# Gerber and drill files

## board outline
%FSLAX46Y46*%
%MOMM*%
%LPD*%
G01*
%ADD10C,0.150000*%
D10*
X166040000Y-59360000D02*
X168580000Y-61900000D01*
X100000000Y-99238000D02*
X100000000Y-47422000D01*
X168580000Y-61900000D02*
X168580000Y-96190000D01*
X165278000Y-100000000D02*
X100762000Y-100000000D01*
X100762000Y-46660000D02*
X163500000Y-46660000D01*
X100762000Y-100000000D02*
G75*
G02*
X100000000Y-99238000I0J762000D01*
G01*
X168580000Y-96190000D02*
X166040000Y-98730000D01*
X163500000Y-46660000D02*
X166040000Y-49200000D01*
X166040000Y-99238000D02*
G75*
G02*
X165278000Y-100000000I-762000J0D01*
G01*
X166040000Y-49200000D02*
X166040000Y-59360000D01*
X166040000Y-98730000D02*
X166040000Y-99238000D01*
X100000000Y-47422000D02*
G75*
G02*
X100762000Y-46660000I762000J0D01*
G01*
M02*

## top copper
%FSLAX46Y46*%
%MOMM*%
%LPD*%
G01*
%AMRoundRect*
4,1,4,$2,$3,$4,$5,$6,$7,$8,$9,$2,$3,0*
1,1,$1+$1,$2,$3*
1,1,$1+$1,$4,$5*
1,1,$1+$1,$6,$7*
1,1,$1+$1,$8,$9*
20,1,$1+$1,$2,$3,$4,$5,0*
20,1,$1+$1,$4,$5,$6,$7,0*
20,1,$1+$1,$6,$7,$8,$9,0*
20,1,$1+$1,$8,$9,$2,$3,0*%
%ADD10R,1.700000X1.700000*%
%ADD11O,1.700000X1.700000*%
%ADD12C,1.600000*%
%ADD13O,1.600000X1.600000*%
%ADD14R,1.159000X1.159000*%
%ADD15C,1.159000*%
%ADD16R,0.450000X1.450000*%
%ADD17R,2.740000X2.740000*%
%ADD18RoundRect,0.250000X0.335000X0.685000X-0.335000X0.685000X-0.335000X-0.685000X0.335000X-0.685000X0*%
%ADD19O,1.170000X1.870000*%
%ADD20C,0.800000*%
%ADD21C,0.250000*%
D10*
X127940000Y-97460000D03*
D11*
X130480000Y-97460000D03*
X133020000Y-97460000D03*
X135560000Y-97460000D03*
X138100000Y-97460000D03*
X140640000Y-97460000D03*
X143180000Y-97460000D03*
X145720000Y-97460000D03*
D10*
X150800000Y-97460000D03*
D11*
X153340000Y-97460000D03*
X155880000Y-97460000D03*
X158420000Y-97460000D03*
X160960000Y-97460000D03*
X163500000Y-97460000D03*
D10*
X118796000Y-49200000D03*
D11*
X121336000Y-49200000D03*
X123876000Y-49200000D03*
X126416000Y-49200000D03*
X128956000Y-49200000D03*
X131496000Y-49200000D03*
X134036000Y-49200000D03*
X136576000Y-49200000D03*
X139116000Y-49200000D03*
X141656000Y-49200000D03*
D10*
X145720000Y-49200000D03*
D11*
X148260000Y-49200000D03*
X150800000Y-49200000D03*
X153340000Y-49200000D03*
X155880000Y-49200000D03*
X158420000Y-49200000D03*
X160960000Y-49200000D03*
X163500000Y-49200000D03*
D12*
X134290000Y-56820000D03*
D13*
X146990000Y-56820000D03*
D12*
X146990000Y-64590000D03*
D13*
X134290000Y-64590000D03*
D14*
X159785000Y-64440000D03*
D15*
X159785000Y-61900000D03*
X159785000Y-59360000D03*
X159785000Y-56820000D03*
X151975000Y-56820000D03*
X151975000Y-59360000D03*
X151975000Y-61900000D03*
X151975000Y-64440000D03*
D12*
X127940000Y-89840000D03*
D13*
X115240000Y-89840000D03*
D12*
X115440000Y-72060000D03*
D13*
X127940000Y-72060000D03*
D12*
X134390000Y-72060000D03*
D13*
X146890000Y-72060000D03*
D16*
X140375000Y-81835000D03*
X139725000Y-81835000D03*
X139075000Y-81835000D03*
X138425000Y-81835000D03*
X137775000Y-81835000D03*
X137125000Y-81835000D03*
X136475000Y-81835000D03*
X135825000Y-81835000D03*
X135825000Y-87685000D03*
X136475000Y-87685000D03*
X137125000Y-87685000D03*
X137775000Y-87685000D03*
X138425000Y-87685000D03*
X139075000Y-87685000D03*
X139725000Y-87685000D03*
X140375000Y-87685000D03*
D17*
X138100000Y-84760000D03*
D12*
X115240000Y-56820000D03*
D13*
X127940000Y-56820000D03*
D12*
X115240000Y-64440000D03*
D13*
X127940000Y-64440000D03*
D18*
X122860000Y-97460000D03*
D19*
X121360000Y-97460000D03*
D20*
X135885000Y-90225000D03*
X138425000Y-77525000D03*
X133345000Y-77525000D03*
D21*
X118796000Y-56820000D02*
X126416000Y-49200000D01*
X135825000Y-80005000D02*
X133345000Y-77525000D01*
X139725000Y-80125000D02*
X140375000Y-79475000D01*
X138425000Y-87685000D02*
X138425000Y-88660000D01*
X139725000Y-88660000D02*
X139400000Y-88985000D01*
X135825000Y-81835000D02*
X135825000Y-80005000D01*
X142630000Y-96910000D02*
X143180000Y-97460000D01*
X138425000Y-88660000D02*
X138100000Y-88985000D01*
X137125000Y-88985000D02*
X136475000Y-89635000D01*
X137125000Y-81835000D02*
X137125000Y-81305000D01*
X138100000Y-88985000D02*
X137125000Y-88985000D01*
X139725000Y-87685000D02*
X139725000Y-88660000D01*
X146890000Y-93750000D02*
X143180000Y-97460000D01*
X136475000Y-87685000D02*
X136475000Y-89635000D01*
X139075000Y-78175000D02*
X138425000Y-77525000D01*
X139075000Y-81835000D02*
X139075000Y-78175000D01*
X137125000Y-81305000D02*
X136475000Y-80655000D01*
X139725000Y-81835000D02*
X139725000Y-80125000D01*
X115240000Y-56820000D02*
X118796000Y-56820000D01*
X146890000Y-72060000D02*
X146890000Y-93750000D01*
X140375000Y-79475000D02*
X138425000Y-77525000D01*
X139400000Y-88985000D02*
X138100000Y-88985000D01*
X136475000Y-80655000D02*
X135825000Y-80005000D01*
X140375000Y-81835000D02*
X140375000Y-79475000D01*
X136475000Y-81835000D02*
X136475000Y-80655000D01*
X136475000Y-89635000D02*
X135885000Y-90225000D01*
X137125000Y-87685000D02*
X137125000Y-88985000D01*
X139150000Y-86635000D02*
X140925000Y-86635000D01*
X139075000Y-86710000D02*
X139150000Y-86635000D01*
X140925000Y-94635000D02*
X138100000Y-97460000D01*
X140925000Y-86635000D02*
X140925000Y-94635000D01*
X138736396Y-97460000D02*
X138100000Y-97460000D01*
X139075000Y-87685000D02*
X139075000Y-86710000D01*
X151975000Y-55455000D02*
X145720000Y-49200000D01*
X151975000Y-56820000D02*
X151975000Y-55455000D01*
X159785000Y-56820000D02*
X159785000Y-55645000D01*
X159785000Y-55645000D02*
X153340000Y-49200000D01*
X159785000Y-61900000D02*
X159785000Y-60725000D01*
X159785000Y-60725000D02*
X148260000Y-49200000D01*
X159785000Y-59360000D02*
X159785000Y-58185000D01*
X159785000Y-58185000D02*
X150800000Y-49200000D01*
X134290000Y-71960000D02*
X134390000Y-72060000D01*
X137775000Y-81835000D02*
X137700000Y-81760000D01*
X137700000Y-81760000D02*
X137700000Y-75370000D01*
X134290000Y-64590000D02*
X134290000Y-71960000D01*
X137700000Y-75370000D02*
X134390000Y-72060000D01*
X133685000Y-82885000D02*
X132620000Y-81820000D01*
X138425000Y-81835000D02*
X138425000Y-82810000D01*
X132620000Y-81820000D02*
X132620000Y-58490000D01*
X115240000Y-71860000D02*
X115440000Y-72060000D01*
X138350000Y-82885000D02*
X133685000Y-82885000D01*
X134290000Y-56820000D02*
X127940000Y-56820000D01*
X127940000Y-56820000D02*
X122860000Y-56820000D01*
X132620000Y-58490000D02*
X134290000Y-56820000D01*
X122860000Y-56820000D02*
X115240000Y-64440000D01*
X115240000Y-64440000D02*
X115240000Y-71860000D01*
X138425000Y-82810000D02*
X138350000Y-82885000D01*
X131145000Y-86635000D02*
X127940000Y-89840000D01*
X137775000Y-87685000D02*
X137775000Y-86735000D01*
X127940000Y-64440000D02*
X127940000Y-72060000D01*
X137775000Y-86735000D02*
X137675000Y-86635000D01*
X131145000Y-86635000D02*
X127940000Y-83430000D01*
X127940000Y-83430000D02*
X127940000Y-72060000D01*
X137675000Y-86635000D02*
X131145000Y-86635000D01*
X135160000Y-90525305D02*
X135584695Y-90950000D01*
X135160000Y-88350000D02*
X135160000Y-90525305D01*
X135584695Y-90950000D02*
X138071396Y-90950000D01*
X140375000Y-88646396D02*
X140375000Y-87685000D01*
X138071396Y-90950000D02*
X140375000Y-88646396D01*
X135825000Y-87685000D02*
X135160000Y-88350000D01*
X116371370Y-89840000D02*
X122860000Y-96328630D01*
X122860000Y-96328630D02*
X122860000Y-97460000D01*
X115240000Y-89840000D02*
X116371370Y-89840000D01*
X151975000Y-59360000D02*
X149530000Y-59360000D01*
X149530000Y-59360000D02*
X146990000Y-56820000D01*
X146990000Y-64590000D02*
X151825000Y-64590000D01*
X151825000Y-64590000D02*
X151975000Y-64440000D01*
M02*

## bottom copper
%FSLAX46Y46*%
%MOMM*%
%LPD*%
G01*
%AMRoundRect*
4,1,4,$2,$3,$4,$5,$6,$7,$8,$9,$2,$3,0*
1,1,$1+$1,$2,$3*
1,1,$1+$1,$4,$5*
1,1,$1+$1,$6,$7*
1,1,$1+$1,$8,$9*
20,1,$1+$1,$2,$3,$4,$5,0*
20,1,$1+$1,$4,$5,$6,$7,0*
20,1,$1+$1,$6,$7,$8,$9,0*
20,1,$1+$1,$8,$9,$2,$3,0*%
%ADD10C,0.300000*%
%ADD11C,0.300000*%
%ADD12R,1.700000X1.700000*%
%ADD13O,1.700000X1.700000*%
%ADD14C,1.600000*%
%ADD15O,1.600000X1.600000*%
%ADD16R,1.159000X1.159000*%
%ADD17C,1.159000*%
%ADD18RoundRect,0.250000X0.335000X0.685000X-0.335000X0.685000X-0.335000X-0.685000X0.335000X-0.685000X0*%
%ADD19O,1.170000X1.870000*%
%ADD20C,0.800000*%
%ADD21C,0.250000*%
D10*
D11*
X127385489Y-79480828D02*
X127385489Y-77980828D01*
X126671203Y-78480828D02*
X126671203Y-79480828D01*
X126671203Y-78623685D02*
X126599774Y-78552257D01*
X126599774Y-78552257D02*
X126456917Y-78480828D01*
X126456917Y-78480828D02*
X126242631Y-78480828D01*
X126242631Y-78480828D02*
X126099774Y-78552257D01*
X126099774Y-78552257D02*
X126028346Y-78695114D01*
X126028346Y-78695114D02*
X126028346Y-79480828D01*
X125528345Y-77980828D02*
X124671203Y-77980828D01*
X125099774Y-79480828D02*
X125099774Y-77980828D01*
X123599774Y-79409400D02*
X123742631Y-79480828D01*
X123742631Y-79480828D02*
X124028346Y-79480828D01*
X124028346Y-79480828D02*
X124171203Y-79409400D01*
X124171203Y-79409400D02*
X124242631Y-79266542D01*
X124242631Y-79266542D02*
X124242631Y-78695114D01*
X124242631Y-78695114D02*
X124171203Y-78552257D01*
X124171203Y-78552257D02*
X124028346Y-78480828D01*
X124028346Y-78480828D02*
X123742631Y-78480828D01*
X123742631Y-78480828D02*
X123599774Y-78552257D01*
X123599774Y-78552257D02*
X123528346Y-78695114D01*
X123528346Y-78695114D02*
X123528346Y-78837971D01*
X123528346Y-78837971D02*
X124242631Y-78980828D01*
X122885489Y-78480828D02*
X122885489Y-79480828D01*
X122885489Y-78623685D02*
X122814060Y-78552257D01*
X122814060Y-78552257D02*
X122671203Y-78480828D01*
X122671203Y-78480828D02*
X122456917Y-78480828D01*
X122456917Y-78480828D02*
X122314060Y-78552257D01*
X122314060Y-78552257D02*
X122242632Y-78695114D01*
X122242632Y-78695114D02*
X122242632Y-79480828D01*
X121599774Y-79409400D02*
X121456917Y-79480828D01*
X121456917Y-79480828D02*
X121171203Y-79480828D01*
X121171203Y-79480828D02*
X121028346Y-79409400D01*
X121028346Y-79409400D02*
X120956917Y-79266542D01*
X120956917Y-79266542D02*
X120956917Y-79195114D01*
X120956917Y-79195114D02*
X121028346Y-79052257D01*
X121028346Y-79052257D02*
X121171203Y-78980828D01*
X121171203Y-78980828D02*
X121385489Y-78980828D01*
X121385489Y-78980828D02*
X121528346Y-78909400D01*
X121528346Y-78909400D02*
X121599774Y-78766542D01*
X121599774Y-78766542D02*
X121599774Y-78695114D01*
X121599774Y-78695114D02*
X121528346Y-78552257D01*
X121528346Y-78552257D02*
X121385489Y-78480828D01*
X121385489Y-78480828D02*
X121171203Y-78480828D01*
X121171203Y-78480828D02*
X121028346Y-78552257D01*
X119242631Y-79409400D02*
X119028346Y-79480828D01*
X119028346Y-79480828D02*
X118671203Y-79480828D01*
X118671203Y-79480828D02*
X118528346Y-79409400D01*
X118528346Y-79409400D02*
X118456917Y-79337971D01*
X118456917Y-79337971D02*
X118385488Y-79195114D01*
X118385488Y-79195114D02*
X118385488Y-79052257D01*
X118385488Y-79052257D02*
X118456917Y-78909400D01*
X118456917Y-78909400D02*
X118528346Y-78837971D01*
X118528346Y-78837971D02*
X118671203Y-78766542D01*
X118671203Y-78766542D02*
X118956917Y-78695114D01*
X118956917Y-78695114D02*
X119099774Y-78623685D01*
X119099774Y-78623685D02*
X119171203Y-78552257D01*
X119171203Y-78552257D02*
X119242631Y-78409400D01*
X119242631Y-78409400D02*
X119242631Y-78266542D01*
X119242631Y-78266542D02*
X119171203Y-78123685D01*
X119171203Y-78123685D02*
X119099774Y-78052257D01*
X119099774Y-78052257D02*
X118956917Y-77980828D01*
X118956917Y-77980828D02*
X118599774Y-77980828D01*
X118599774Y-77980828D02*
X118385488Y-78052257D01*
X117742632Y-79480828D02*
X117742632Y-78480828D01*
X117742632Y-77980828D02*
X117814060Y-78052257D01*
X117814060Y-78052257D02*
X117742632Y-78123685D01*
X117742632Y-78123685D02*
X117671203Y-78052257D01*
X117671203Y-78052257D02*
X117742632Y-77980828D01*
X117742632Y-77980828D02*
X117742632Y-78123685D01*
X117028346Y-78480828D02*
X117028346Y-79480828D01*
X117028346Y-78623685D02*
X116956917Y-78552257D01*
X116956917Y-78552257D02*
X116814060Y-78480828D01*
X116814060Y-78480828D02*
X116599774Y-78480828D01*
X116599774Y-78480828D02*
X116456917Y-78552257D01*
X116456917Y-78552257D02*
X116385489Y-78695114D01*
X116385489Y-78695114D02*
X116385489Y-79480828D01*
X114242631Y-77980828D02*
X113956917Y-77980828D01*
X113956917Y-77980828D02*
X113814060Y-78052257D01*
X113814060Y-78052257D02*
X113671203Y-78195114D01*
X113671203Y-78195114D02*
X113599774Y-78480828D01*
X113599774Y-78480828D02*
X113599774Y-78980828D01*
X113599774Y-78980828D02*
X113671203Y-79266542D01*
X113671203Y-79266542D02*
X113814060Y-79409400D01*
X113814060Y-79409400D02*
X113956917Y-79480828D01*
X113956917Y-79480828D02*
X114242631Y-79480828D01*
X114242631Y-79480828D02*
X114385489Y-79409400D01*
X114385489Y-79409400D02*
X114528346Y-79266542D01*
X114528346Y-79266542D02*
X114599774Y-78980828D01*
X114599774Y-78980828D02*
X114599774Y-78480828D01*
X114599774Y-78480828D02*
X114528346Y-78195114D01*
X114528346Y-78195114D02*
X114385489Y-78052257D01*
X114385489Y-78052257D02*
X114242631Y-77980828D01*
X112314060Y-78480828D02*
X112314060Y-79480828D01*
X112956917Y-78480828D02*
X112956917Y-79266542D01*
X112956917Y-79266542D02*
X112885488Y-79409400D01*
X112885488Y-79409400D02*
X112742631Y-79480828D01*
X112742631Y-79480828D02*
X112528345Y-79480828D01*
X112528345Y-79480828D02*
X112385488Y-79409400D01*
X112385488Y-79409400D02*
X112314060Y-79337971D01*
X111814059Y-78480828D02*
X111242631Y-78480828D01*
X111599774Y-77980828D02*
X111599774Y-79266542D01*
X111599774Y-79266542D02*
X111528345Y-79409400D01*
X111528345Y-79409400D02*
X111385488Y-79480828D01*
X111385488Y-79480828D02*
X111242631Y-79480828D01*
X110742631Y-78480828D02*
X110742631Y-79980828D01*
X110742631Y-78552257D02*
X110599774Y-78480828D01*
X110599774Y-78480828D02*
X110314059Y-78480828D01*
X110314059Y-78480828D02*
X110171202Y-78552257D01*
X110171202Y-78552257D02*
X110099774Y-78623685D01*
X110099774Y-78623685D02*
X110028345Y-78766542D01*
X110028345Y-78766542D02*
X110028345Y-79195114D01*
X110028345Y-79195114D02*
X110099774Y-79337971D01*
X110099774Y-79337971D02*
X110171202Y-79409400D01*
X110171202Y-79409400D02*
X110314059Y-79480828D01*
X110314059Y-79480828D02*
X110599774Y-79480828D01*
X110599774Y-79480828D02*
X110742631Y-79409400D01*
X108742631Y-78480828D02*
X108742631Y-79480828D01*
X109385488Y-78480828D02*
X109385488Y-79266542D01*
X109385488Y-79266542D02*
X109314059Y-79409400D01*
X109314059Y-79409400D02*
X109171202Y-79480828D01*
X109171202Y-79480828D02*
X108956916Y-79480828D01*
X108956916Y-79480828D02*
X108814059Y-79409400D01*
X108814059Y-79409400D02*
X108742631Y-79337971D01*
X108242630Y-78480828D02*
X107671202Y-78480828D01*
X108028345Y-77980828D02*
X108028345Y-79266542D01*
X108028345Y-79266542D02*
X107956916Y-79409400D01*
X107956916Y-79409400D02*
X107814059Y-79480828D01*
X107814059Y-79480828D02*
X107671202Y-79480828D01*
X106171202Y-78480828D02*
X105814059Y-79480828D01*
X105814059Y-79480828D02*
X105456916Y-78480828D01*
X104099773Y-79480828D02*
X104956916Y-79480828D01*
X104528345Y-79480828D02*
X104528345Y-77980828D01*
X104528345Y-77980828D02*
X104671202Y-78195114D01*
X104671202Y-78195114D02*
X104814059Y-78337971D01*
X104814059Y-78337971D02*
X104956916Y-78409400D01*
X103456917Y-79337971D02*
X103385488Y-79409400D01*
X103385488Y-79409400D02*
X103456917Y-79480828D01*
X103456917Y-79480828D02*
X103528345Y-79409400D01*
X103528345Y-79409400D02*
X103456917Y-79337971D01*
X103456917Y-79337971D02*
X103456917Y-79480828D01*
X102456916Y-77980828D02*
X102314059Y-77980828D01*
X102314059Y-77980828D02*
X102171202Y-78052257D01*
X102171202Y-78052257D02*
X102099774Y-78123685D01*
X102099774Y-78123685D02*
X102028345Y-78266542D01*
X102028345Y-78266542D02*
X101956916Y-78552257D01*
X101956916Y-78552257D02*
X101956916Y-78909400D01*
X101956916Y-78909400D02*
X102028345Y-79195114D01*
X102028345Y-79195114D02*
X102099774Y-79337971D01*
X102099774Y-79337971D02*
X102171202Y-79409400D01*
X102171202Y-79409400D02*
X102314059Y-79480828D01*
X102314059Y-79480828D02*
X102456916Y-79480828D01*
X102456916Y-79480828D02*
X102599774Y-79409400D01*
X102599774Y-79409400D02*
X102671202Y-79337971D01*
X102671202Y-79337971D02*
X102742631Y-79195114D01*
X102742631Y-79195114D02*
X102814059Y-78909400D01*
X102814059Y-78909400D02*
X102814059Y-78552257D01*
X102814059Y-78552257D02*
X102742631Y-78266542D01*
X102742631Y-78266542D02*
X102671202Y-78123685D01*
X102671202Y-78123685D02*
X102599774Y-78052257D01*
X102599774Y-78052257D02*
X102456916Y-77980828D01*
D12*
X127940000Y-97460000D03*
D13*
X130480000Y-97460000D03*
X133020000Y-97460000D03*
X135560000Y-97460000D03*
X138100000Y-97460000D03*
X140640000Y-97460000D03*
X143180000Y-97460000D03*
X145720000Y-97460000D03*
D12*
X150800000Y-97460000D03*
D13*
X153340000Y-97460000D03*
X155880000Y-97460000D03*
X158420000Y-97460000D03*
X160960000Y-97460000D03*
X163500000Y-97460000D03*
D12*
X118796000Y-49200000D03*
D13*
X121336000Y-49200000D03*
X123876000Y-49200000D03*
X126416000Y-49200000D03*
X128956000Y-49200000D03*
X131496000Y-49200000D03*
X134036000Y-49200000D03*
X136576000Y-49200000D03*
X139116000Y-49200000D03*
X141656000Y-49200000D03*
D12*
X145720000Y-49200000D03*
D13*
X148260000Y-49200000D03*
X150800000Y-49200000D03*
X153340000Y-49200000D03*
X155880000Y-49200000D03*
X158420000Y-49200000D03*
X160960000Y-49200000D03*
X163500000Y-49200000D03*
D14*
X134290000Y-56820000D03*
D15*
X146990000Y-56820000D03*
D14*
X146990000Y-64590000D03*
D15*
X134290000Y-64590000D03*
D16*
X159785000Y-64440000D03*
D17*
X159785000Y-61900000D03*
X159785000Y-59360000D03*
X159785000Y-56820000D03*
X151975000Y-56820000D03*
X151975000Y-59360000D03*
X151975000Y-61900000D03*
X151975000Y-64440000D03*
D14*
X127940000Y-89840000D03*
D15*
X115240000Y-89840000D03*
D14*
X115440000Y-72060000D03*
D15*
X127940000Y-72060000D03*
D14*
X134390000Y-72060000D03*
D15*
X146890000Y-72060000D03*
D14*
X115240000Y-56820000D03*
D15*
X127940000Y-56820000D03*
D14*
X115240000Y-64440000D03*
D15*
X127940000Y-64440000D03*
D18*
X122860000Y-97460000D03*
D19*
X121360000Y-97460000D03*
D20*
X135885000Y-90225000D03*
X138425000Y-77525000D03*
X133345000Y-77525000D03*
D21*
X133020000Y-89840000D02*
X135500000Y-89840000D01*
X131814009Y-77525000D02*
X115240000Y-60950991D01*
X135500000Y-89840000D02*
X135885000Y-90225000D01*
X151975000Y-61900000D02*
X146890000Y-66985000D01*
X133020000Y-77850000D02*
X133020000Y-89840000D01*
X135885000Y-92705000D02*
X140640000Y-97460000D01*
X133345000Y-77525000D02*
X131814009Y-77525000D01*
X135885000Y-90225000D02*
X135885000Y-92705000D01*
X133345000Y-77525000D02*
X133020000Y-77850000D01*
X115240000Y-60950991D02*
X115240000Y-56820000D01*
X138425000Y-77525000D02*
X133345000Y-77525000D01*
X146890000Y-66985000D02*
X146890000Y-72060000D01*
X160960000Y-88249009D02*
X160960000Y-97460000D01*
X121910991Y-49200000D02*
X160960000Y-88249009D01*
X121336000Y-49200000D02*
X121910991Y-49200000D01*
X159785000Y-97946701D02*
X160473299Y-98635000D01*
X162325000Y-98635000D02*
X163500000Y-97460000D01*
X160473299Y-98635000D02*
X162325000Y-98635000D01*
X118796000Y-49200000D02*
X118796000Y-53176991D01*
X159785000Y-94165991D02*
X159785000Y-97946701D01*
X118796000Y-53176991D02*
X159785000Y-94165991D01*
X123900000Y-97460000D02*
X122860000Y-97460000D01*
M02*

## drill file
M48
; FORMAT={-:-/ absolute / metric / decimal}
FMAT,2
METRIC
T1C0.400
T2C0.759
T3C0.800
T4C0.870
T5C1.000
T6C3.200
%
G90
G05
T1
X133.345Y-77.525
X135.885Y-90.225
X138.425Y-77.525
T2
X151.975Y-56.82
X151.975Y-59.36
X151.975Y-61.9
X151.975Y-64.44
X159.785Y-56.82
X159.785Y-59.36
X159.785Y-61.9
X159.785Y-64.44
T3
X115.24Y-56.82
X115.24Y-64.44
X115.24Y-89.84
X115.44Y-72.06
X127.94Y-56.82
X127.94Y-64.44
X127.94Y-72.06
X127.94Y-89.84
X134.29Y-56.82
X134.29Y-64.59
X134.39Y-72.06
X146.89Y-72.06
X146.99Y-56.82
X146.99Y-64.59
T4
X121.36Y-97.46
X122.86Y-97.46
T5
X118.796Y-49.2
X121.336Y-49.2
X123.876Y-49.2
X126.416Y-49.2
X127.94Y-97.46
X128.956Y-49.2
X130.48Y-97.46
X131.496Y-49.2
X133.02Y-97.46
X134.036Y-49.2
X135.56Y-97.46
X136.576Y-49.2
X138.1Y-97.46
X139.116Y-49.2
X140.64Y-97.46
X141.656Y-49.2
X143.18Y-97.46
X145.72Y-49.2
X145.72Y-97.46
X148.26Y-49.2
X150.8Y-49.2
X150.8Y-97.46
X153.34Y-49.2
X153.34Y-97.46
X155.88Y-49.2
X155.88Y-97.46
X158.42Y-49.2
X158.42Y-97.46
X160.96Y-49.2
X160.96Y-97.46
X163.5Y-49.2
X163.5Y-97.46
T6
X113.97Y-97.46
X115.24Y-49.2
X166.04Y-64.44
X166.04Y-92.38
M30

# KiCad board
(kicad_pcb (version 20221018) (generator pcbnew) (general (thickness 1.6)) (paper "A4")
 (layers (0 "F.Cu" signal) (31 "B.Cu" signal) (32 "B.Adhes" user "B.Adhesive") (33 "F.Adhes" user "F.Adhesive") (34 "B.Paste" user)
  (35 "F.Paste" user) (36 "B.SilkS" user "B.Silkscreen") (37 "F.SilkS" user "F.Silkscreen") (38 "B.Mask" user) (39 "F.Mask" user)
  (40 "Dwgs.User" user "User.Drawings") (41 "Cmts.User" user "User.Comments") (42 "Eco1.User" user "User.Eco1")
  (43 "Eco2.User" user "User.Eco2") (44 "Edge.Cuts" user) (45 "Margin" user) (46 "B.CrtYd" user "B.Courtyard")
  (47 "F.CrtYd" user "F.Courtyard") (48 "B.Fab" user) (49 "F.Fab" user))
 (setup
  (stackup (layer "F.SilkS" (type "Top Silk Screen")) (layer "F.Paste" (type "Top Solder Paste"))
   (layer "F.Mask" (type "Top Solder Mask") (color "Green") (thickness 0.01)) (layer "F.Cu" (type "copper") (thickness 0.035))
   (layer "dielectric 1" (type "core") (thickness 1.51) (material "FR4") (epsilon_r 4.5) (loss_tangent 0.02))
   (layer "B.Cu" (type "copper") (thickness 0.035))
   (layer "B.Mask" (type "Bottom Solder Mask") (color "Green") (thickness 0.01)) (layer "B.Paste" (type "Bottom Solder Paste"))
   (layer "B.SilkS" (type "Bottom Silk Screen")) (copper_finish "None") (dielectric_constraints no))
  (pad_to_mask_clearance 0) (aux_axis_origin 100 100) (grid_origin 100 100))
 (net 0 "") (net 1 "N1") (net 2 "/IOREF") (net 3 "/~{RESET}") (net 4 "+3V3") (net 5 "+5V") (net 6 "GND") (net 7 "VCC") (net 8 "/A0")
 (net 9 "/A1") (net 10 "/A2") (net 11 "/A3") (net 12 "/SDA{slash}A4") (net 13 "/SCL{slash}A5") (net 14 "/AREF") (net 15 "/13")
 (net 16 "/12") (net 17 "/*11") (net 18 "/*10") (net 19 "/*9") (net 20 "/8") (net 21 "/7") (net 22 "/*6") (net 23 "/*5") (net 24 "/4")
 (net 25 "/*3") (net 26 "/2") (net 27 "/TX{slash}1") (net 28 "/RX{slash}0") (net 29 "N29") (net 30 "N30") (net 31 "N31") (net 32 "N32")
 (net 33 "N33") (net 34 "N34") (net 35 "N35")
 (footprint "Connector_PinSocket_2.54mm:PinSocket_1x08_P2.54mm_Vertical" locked (layer "F.Cu") (at 127.94 97.46 90)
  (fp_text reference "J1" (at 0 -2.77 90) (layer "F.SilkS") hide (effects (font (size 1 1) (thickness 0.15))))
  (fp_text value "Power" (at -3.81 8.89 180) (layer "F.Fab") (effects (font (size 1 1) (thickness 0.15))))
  (pad "1" thru_hole rect locked (at 0 0 90) (size 1.7 1.7) (drill 1) (layers "*.Cu" "*.Mask") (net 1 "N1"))
  (pad "2" thru_hole oval locked (at 0 2.54 90) (size 1.7 1.7) (drill 1) (layers "*.Cu" "*.Mask") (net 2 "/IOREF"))
  (pad "3" thru_hole oval locked (at 0 5.08 90) (size 1.7 1.7) (drill 1) (layers "*.Cu" "*.Mask") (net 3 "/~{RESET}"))
  (pad "4" thru_hole oval locked (at 0 7.62 90) (size 1.7 1.7) (drill 1) (layers "*.Cu" "*.Mask") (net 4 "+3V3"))
  (pad "5" thru_hole oval locked (at 0 10.16 90) (size 1.7 1.7) (drill 1) (layers "*.Cu" "*.Mask") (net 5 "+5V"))
  (pad "6" thru_hole oval locked (at 0 12.7 90) (size 1.7 1.7) (drill 1) (layers "*.Cu" "*.Mask") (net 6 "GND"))
  (pad "7" thru_hole oval locked (at 0 15.24 90) (size 1.7 1.7) (drill 1) (layers "*.Cu" "*.Mask") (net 6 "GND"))
  (pad "8" thru_hole oval locked (at 0 17.78 90) (size 1.7 1.7) (drill 1) (layers "*.Cu" "*.Mask") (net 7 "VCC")))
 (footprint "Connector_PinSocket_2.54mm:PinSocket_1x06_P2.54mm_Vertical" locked (layer "F.Cu") (at 150.8 97.46 90)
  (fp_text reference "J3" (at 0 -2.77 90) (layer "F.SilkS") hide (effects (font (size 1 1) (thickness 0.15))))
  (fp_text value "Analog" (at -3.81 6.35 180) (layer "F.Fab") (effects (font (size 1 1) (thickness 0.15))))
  (pad "1" thru_hole rect locked (at 0 0 90) (size 1.7 1.7) (drill 1) (layers "*.Cu" "*.Mask") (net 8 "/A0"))
  (pad "2" thru_hole oval locked (at 0 2.54 90) (size 1.7 1.7) (drill 1) (layers "*.Cu" "*.Mask") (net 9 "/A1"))
  (pad "3" thru_hole oval locked (at 0 5.08 90) (size 1.7 1.7) (drill 1) (layers "*.Cu" "*.Mask") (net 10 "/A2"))
  (pad "4" thru_hole oval locked (at 0 7.62 90) (size 1.7 1.7) (drill 1) (layers "*.Cu" "*.Mask") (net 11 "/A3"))
  (pad "5" thru_hole oval locked (at 0 10.16 90) (size 1.7 1.7) (drill 1) (layers "*.Cu" "*.Mask") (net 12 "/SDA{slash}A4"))
  (pad "6" thru_hole oval locked (at 0 12.7 90) (size 1.7 1.7) (drill 1) (layers "*.Cu" "*.Mask") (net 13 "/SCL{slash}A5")))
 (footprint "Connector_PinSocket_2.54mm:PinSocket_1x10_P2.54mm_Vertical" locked (layer "F.Cu") (at 118.796 49.2 90)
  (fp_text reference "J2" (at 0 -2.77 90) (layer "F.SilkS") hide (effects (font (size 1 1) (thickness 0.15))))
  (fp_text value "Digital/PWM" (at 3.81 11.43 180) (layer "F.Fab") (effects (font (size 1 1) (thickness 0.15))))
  (pad "1" thru_hole rect locked (at 0 0 90) (size 1.7 1.7) (drill 1) (layers "*.Cu" "*.Mask") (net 13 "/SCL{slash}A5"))
  (pad "2" thru_hole oval locked (at 0 2.54 90) (size 1.7 1.7) (drill 1) (layers "*.Cu" "*.Mask") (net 12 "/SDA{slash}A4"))
  (pad "3" thru_hole oval locked (at 0 5.08 90) (size 1.7 1.7) (drill 1) (layers "*.Cu" "*.Mask") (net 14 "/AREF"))
  (pad "4" thru_hole oval locked (at 0 7.62 90) (size 1.7 1.7) (drill 1) (layers "*.Cu" "*.Mask") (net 6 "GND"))
  (pad "5" thru_hole oval locked (at 0 10.16 90) (size 1.7 1.7) (drill 1) (layers "*.Cu" "*.Mask") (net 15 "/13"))
  (pad "6" thru_hole oval locked (at 0 12.7 90) (size 1.7 1.7) (drill 1) (layers "*.Cu" "*.Mask") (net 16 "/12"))
  (pad "7" thru_hole oval locked (at 0 15.24 90) (size 1.7 1.7) (drill 1) (layers "*.Cu" "*.Mask") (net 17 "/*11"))
  (pad "8" thru_hole oval locked (at 0 17.78 90) (size 1.7 1.7) (drill 1) (layers "*.Cu" "*.Mask") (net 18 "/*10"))
  (pad "9" thru_hole oval locked (at 0 20.32 90) (size 1.7 1.7) (drill 1) (layers "*.Cu" "*.Mask") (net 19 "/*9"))
  (pad "10" thru_hole oval locked (at 0 22.86 90) (size 1.7 1.7) (drill 1) (layers "*.Cu" "*.Mask") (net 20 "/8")))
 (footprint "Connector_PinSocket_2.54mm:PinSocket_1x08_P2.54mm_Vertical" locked (layer "F.Cu") (at 145.72 49.2 90)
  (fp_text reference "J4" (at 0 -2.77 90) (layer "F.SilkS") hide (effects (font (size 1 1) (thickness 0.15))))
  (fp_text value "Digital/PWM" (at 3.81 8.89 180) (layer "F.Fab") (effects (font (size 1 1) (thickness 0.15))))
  (pad "1" thru_hole rect locked (at 0 0 90) (size 1.7 1.7) (drill 1) (layers "*.Cu" "*.Mask") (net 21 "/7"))
  (pad "2" thru_hole oval locked (at 0 2.54 90) (size 1.7 1.7) (drill 1) (layers "*.Cu" "*.Mask") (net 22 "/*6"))
  (pad "3" thru_hole oval locked (at 0 5.08 90) (size 1.7 1.7) (drill 1) (layers "*.Cu" "*.Mask") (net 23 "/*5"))
  (pad "4" thru_hole oval locked (at 0 7.62 90) (size 1.7 1.7) (drill 1) (layers "*.Cu" "*.Mask") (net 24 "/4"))
  (pad "5" thru_hole oval locked (at 0 10.16 90) (size 1.7 1.7) (drill 1) (layers "*.Cu" "*.Mask") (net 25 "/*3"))
  (pad "6" thru_hole oval locked (at 0 12.7 90) (size 1.7 1.7) (drill 1) (layers "*.Cu" "*.Mask") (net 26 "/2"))
  (pad "7" thru_hole oval locked (at 0 15.24 90) (size 1.7 1.7) (drill 1) (layers "*.Cu" "*.Mask") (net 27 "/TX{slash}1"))
  (pad "8" thru_hole oval locked (at 0 17.78 90) (size 1.7 1.7) (drill 1) (layers "*.Cu" "*.Mask") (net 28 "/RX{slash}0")))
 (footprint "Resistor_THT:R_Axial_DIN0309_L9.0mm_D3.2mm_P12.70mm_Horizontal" (layer "F.Cu") (at 134.29 56.82)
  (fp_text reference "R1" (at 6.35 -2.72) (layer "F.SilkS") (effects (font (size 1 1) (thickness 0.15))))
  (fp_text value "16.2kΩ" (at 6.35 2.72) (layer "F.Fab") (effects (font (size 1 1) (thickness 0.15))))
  (pad "1" thru_hole circle (at 0 0) (size 1.6 1.6) (drill 0.8) (layers "*.Cu" "*.Mask") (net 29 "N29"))
  (pad "2" thru_hole oval (at 12.7 0) (size 1.6 1.6) (drill 0.8) (layers "*.Cu" "*.Mask") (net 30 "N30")))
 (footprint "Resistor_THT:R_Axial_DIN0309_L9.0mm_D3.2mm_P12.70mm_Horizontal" (layer "F.Cu") (at 146.99 64.59 180)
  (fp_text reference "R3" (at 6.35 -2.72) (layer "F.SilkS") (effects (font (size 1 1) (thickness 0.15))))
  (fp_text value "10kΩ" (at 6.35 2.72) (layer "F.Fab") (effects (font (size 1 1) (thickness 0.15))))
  (pad "1" thru_hole circle (at 0 0 180) (size 1.6 1.6) (drill 0.8) (layers "*.Cu" "*.Mask") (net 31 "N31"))
  (pad "2" thru_hole oval (at 12.7 0 180) (size 1.6 1.6) (drill 0.8) (layers "*.Cu" "*.Mask") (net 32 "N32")))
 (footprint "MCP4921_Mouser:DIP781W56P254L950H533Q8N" (layer "F.Cu") (at 155.88 60.63 180)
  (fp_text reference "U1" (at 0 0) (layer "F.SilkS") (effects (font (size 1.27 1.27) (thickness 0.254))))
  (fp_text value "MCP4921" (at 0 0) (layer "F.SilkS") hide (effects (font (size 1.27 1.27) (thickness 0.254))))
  (pad "1" thru_hole rect (at -3.905 -3.81 180) (size 1.159 1.159) (drill 0.759) (layers "*.Cu" "*.Mask") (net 5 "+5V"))
  (pad "2" thru_hole circle (at -3.905 -1.27 180) (size 1.159 1.159) (drill 0.759) (layers "*.Cu" "*.Mask") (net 22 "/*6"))
  (pad "3" thru_hole circle (at -3.905 1.27 180) (size 1.159 1.159) (drill 0.759) (layers "*.Cu" "*.Mask") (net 23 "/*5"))
  (pad "4" thru_hole circle (at -3.905 3.81 180) (size 1.159 1.159) (drill 0.759) (layers "*.Cu" "*.Mask") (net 24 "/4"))
  (pad "5" thru_hole circle (at 3.905 3.81 180) (size 1.159 1.159) (drill 0.759) (layers "*.Cu" "*.Mask") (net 21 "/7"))
  (pad "6" thru_hole circle (at 3.905 1.27 180) (size 1.159 1.159) (drill 0.759) (layers "*.Cu" "*.Mask") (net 30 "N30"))
  (pad "7" thru_hole circle (at 3.905 -1.27 180) (size 1.159 1.159) (drill 0.759) (layers "*.Cu" "*.Mask") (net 6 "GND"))
  (pad "8" thru_hole circle (at 3.905 -3.81 180) (size 1.159 1.159) (drill 0.759) (layers "*.Cu" "*.Mask") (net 31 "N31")))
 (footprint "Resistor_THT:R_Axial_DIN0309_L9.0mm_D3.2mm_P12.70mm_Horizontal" (layer "F.Cu") (at 127.94 89.84 180)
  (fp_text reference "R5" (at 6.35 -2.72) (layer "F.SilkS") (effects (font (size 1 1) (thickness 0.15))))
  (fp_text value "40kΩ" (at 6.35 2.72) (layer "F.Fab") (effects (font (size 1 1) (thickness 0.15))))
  (pad "1" thru_hole circle (at 0 0 180) (size 1.6 1.6) (drill 0.8) (layers "*.Cu" "*.Mask") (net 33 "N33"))
  (pad "2" thru_hole oval (at 12.7 0 180) (size 1.6 1.6) (drill 0.8) (layers "*.Cu" "*.Mask") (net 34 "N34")))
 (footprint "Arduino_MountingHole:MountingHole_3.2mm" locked (layer "F.Cu") (at 115.24 49.2)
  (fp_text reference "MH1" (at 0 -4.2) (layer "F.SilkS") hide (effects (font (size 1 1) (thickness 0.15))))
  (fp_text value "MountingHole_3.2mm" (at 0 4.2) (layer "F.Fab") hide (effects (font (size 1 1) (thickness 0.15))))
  (pad "" np_thru_hole circle locked (at 0 0) (size 3.2 3.2) (drill 3.2) (layers "*.Cu" "*.Mask")))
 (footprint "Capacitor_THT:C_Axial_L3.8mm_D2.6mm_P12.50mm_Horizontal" (layer "F.Cu") (at 115.44 72.06)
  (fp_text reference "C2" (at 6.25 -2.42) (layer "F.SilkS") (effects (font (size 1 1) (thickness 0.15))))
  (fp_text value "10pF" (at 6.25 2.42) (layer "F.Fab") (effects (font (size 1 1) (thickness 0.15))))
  (pad "1" thru_hole circle (at 0 0) (size 1.6 1.6) (drill 0.8) (layers "*.Cu" "*.Mask") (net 29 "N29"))
  (pad "2" thru_hole oval (at 12.5 0) (size 1.6 1.6) (drill 0.8) (layers "*.Cu" "*.Mask") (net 33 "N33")))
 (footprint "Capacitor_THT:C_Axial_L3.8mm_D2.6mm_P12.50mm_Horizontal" (layer "F.Cu") (at 134.39 72.06)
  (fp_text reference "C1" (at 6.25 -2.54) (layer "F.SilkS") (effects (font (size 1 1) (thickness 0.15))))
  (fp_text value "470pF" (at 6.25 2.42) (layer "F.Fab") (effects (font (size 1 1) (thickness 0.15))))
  (pad "1" thru_hole circle (at 0 0) (size 1.6 1.6) (drill 0.8) (layers "*.Cu" "*.Mask") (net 32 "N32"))
  (pad "2" thru_hole oval (at 12.5 0) (size 1.6 1.6) (drill 0.8) (layers "*.Cu" "*.Mask") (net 6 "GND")))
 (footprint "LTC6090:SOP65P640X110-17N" (layer "F.Cu") (at 138.1 84.76 -90)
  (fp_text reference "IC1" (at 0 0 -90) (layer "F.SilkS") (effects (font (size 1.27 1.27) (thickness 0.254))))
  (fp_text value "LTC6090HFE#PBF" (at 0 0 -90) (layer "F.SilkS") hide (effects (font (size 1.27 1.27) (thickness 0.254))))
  (pad "1" smd rect (at -2.925 -2.275) (size 0.45 1.45) (layers "F.Cu" "F.Paste" "F.Mask") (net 6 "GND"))
  (pad "2" smd rect (at -2.925 -1.625) (size 0.45 1.45) (layers "F.Cu" "F.Paste" "F.Mask") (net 6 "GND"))
  (pad "3" smd rect (at -2.925 -0.975) (size 0.45 1.45) (layers "F.Cu" "F.Paste" "F.Mask") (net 6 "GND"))
  (pad "4" smd rect (at -2.925 -0.325) (size 0.45 1.45) (layers "F.Cu" "F.Paste" "F.Mask") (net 29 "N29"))
  (pad "5" smd rect (at -2.925 0.325) (size 0.45 1.45) (layers "F.Cu" "F.Paste" "F.Mask") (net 32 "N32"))
  (pad "6" smd rect (at -2.925 0.975) (size 0.45 1.45) (layers "F.Cu" "F.Paste" "F.Mask") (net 6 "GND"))
  (pad "7" smd rect (at -2.925 1.625) (size 0.45 1.45) (layers "F.Cu" "F.Paste" "F.Mask") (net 6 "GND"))
  (pad "8" smd rect (at -2.925 2.275) (size 0.45 1.45) (layers "F.Cu" "F.Paste" "F.Mask") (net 6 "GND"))
  (pad "9" smd rect (at 2.925 2.275) (size 0.45 1.45) (layers "F.Cu" "F.Paste" "F.Mask") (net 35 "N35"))
  (pad "10" smd rect (at 2.925 1.625) (size 0.45 1.45) (layers "F.Cu" "F.Paste" "F.Mask") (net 6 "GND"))
  (pad "11" smd rect (at 2.925 0.975) (size 0.45 1.45) (layers "F.Cu" "F.Paste" "F.Mask") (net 6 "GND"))
  (pad "12" smd rect (at 2.925 0.325) (size 0.45 1.45) (layers "F.Cu" "F.Paste" "F.Mask") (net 33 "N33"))
  (pad "13" smd rect (at 2.925 -0.325) (size 0.45 1.45) (layers "F.Cu" "F.Paste" "F.Mask") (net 6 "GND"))
  (pad "14" smd rect (at 2.925 -0.975) (size 0.45 1.45) (layers "F.Cu" "F.Paste" "F.Mask") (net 5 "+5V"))
  (pad "15" smd rect (at 2.925 -1.625) (size 0.45 1.45) (layers "F.Cu" "F.Paste" "F.Mask") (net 6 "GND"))
  (pad "16" smd rect (at 2.925 -2.275) (size 0.45 1.45) (layers "F.Cu" "F.Paste" "F.Mask") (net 35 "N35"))
  (pad "17" smd rect (at 0 0 270) (size 2.74 2.74) (layers "F.Cu" "F.Paste" "F.Mask") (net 6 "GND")))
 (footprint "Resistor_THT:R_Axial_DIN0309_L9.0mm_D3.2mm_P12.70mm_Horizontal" (layer "F.Cu") (at 115.24 56.82)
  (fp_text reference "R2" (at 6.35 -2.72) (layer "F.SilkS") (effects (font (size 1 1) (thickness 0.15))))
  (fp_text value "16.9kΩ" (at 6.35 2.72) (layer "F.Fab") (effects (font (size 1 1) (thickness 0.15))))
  (pad "1" thru_hole circle (at 0 0) (size 1.6 1.6) (drill 0.8) (layers "*.Cu" "*.Mask") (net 6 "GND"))
  (pad "2" thru_hole oval (at 12.7 0) (size 1.6 1.6) (drill 0.8) (layers "*.Cu" "*.Mask") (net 29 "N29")))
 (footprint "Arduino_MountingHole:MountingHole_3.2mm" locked (layer "F.Cu") (at 113.97 97.46)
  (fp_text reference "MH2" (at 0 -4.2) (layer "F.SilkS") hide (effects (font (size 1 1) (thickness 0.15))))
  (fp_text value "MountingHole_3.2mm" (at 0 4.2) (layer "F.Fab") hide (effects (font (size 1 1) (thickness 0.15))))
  (pad "" np_thru_hole circle locked (at 0 0) (size 3.2 3.2) (drill 3.2) (layers "*.Cu" "*.Mask")))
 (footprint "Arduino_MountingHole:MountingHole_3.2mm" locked (layer "F.Cu") (at 166.04 64.44)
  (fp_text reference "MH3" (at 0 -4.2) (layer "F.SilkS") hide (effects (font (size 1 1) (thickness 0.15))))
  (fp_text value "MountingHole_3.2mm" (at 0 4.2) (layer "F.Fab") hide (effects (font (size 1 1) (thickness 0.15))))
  (pad "" np_thru_hole circle locked (at 0 0) (size 3.2 3.2) (drill 3.2) (layers "*.Cu" "*.Mask")))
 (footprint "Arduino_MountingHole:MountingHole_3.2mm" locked (layer "F.Cu") (at 166.04 92.38)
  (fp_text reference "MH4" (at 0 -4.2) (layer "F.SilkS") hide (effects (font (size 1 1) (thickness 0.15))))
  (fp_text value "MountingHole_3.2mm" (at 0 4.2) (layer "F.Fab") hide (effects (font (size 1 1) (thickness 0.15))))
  (pad "" np_thru_hole circle locked (at 0 0) (size 3.2 3.2) (drill 3.2) (layers "*.Cu" "*.Mask")))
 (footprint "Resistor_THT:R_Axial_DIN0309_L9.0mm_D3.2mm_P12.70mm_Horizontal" (layer "F.Cu") (at 115.24 64.44)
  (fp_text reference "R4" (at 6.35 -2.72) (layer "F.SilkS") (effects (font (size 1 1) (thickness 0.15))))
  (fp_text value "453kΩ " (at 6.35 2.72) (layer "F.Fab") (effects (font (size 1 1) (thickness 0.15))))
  (pad "1" thru_hole circle (at 0 0) (size 1.6 1.6) (drill 0.8) (layers "*.Cu" "*.Mask") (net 29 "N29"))
  (pad "2" thru_hole oval (at 12.7 0) (size 1.6 1.6) (drill 0.8) (layers "*.Cu" "*.Mask") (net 33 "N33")))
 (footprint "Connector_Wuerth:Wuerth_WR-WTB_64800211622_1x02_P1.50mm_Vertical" (layer "B.Cu") (at 122.86 97.46 180)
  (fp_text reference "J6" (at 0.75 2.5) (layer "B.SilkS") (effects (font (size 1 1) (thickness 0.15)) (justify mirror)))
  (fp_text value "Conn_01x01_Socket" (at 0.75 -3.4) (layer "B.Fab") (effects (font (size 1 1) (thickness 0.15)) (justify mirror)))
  (pad "1" thru_hole roundrect (at 0 0 180) (size 1.17 1.87) (drill 0.87) (layers "*.Cu" "*.Mask") (roundrect_rratio 0.213675)
   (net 34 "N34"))
  (pad "2" thru_hole oval (at 1.5 0 180) (size 1.17 1.87) (drill 0.87) (layers "*.Cu" "*.Mask")))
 (gr_line (start 166.04 59.36) (end 168.58 61.9) (stroke (width 0.15) (type solid)) (layer "Edge.Cuts"))
 (gr_line (start 100 99.238) (end 100 47.422) (stroke (width 0.15) (type solid)) (layer "Edge.Cuts"))
 (gr_line (start 168.58 61.9) (end 168.58 96.19) (stroke (width 0.15) (type solid)) (layer "Edge.Cuts"))
 (gr_line (start 165.278 100) (end 100.762 100) (stroke (width 0.15) (type solid)) (layer "Edge.Cuts"))
 (gr_line (start 100.762 46.66) (end 163.5 46.66) (stroke (width 0.15) (type solid)) (layer "Edge.Cuts"))
 (gr_arc (start 100.762 100) (mid 100.223185 99.776815) (end 100 99.238) (stroke (width 0.15) (type solid)) (layer "Edge.Cuts"))
 (gr_line (start 168.58 96.19) (end 166.04 98.73) (stroke (width 0.15) (type solid)) (layer "Edge.Cuts"))
 (gr_line (start 163.5 46.66) (end 166.04 49.2) (stroke (width 0.15) (type solid)) (layer "Edge.Cuts"))
 (gr_arc (start 166.04 99.238) (mid 165.816815 99.776815) (end 165.278 100) (stroke (width 0.15) (type solid)) (layer "Edge.Cuts"))
 (gr_line (start 166.04 49.2) (end 166.04 59.36) (stroke (width 0.15) (type solid)) (layer "Edge.Cuts"))
 (gr_line (start 166.04 98.73) (end 166.04 99.238) (stroke (width 0.15) (type solid)) (layer "Edge.Cuts"))
 (gr_arc (start 100 47.422) (mid 100.223185 46.883185) (end 100.762 46.66) (stroke (width 0.15) (type solid)) (layer "Edge.Cuts"))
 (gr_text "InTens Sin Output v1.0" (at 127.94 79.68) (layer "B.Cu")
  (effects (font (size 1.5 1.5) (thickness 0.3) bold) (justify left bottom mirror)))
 (segment (start 118.796 56.82) (end 126.416 49.2) (width 0.25) (layer "F.Cu") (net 6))
 (segment (start 135.825 80.005) (end 133.345 77.525) (width 0.25) (layer "F.Cu") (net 6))
 (segment (start 139.725 80.125) (end 140.375 79.475) (width 0.25) (layer "F.Cu") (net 6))
 (segment (start 138.425 87.685) (end 138.425 88.66) (width 0.25) (layer "F.Cu") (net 6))
 (segment (start 139.725 88.66) (end 139.4 88.985) (width 0.25) (layer "F.Cu") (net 6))
 (segment (start 135.825 81.835) (end 135.825 80.005) (width 0.25) (layer "F.Cu") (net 6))
 (segment (start 142.63 96.91) (end 143.18 97.46) (width 0.25) (layer "F.Cu") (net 6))
 (segment (start 138.425 88.66) (end 138.1 88.985) (width 0.25) (layer "F.Cu") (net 6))
 (segment (start 137.125 88.985) (end 136.475 89.635) (width 0.25) (layer "F.Cu") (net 6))
 (segment (start 137.125 81.835) (end 137.125 81.305) (width 0.25) (layer "F.Cu") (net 6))
 (segment (start 138.1 88.985) (end 137.125 88.985) (width 0.25) (layer "F.Cu") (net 6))
 (segment (start 139.725 87.685) (end 139.725 88.66) (width 0.25) (layer "F.Cu") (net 6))
 (segment (start 146.89 93.75) (end 143.18 97.46) (width 0.25) (layer "F.Cu") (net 6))
 (segment (start 136.475 87.685) (end 136.475 89.635) (width 0.25) (layer "F.Cu") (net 6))
 (segment (start 139.075 78.175) (end 138.425 77.525) (width 0.25) (layer "F.Cu") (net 6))
 (segment (start 139.075 81.835) (end 139.075 78.175) (width 0.25) (layer "F.Cu") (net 6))
 (segment (start 137.125 81.305) (end 136.475 80.655) (width 0.25) (layer "F.Cu") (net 6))
 (segment (start 139.725 81.835) (end 139.725 80.125) (width 0.25) (layer "F.Cu") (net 6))
 (segment (start 115.24 56.82) (end 118.796 56.82) (width 0.25) (layer "F.Cu") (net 6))
 (segment (start 146.89 72.06) (end 146.89 93.75) (width 0.25) (layer "F.Cu") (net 6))
 (segment (start 140.375 79.475) (end 138.425 77.525) (width 0.25) (layer "F.Cu") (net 6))
 (segment (start 139.4 88.985) (end 138.1 88.985) (width 0.25) (layer "F.Cu") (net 6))
 (segment (start 136.475 80.655) (end 135.825 80.005) (width 0.25) (layer "F.Cu") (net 6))
 (segment (start 140.375 81.835) (end 140.375 79.475) (width 0.25) (layer "F.Cu") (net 6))
 (segment (start 136.475 81.835) (end 136.475 80.655) (width 0.25) (layer "F.Cu") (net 6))
 (segment (start 136.475 89.635) (end 135.885 90.225) (width 0.25) (layer "F.Cu") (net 6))
 (segment (start 137.125 87.685) (end 137.125 88.985) (width 0.25) (layer "F.Cu") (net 6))
 (via (at 135.885 90.225) (size 0.8) (drill 0.4) (layers "F.Cu" "B.Cu") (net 6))
 (via (at 138.425 77.525) (size 0.8) (drill 0.4) (layers "F.Cu" "B.Cu") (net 6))
 (via (at 133.345 77.525) (size 0.8) (drill 0.4) (layers "F.Cu" "B.Cu") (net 6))
 (segment (start 133.02 89.84) (end 135.5 89.84) (width 0.25) (layer "B.Cu") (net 6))
 (segment (start 131.814009 77.525) (end 115.24 60.950991) (width 0.25) (layer "B.Cu") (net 6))
 (segment (start 135.5 89.84) (end 135.885 90.225) (width 0.25) (layer "B.Cu") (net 6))
 (segment (start 151.975 61.9) (end 146.89 66.985) (width 0.25) (layer "B.Cu") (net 6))
 (segment (start 133.02 77.85) (end 133.02 89.84) (width 0.25) (layer "B.Cu") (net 6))
 (segment (start 135.885 92.705) (end 140.64 97.46) (width 0.25) (layer "B.Cu") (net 6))
 (segment (start 133.345 77.525) (end 131.814009 77.525) (width 0.25) (layer "B.Cu") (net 6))
 (segment (start 135.885 90.225) (end 135.885 92.705) (width 0.25) (layer "B.Cu") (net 6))
 (segment (start 133.345 77.525) (end 133.02 77.85) (width 0.25) (layer "B.Cu") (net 6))
 (segment (start 115.24 60.950991) (end 115.24 56.82) (width 0.25) (layer "B.Cu") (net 6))
 (segment (start 138.425 77.525) (end 133.345 77.525) (width 0.25) (layer "B.Cu") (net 6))
 (segment (start 146.89 66.985) (end 146.89 72.06) (width 0.25) (layer "B.Cu") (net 6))
 (segment (start 139.15 86.635) (end 140.925 86.635) (width 0.25) (layer "F.Cu") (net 5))
 (segment (start 139.075 86.71) (end 139.15 86.635) (width 0.25) (layer "F.Cu") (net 5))
 (segment (start 140.925 94.635) (end 138.1 97.46) (width 0.25) (layer "F.Cu") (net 5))
 (segment (start 140.925 86.635) (end 140.925 94.635) (width 0.25) (layer "F.Cu") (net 5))
 (segment (start 138.736396 97.46) (end 138.1 97.46) (width 0.25) (layer "F.Cu") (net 5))
 (segment (start 139.075 87.685) (end 139.075 86.71) (width 0.25) (layer "F.Cu") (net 5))
 (segment (start 160.96 88.249009) (end 160.96 97.46) (width 0.25) (layer "B.Cu") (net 12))
 (segment (start 121.910991 49.2) (end 160.96 88.249009) (width 0.25) (layer "B.Cu") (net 12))
 (segment (start 121.336 49.2) (end 121.910991 49.2) (width 0.25) (layer "B.Cu") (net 12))
 (segment (start 159.785 97.946701) (end 160.473299 98.635) (width 0.25) (layer "B.Cu") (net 13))
 (segment (start 162.325 98.635) (end 163.5 97.46) (width 0.25) (layer "B.Cu") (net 13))
 (segment (start 160.473299 98.635) (end 162.325 98.635) (width 0.25) (layer "B.Cu") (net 13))
 (segment (start 118.796 49.2) (end 118.796 53.176991) (width 0.25) (layer "B.Cu") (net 13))
 (segment (start 159.785 94.165991) (end 159.785 97.946701) (width 0.25) (layer "B.Cu") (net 13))
 (segment (start 118.796 53.176991) (end 159.785 94.165991) (width 0.25) (layer "B.Cu") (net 13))
 (segment (start 151.975 55.455) (end 145.72 49.2) (width 0.25) (layer "F.Cu") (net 21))
 (segment (start 151.975 56.82) (end 151.975 55.455) (width 0.25) (layer "F.Cu") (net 21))
 (segment (start 159.785 56.82) (end 159.785 55.645) (width 0.25) (layer "F.Cu") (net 24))
 (segment (start 159.785 55.645) (end 153.34 49.2) (width 0.25) (layer "F.Cu") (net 24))
 (segment (start 159.785 61.9) (end 159.785 60.725) (width 0.25) (layer "F.Cu") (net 22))
 (segment (start 159.785 60.725) (end 148.26 49.2) (width 0.25) (layer "F.Cu") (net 22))
 (segment (start 159.785 59.36) (end 159.785 58.185) (width 0.25) (layer "F.Cu") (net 23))
 (segment (start 159.785 58.185) (end 150.8 49.2) (width 0.25) (layer "F.Cu") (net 23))
 (segment (start 134.29 71.96) (end 134.39 72.06) (width 0.25) (layer "F.Cu") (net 32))
 (segment (start 137.775 81.835) (end 137.7 81.76) (width 0.25) (layer "F.Cu") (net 32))
 (segment (start 137.7 81.76) (end 137.7 75.37) (width 0.25) (layer "F.Cu") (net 32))
 (segment (start 134.29 64.59) (end 134.29 71.96) (width 0.25) (layer "F.Cu") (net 32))
 (segment (start 137.7 75.37) (end 134.39 72.06) (width 0.25) (layer "F.Cu") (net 32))
 (segment (start 133.685 82.885) (end 132.62 81.82) (width 0.25) (layer "F.Cu") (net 29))
 (segment (start 138.425 81.835) (end 138.425 82.81) (width 0.25) (layer "F.Cu") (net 29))
 (segment (start 132.62 81.82) (end 132.62 58.49) (width 0.25) (layer "F.Cu") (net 29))
 (segment (start 115.24 71.86) (end 115.44 72.06) (width 0.25) (layer "F.Cu") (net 29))
 (segment (start 138.35 82.885) (end 133.685 82.885) (width 0.25) (layer "F.Cu") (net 29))
 (segment (start 134.29 56.82) (end 127.94 56.82) (width 0.25) (layer "F.Cu") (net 29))
 (segment (start 127.94 56.82) (end 122.86 56.82) (width 0.25) (layer "F.Cu") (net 29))
 (segment (start 132.62 58.49) (end 134.29 56.82) (width 0.25) (layer "F.Cu") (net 29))
 (segment (start 122.86 56.82) (end 115.24 64.44) (width 0.25) (layer "F.Cu") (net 29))
 (segment (start 115.24 64.44) (end 115.24 71.86) (width 0.25) (layer "F.Cu") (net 29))
 (segment (start 138.425 82.81) (end 138.35 82.885) (width 0.25) (layer "F.Cu") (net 29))
 (segment (start 131.145 86.635) (end 127.94 89.84) (width 0.25) (layer "F.Cu") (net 33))
 (segment (start 137.775 87.685) (end 137.775 86.735) (width 0.25) (layer "F.Cu") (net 33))
 (segment (start 127.94 64.44) (end 127.94 72.06) (width 0.25) (layer "F.Cu") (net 33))
 (segment (start 137.775 86.735) (end 137.675 86.635) (width 0.25) (layer "F.Cu") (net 33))
 (segment (start 131.145 86.635) (end 127.94 83.43) (width 0.25) (layer "F.Cu") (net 33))
 (segment (start 127.94 83.43) (end 127.94 72.06) (width 0.25) (layer "F.Cu") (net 33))
 (segment (start 137.675 86.635) (end 131.145 86.635) (width 0.25) (layer "F.Cu") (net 33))
 (segment (start 135.16 90.525305) (end 135.584695 90.95) (width 0.25) (layer "F.Cu") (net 35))
 (segment (start 135.16 88.35) (end 135.16 90.525305) (width 0.25) (layer "F.Cu") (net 35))
 (segment (start 135.584695 90.95) (end 138.071396 90.95) (width 0.25) (layer "F.Cu") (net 35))
 (segment (start 140.375 88.646396) (end 140.375 87.685) (width 0.25) (layer "F.Cu") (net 35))
 (segment (start 138.071396 90.95) (end 140.375 88.646396) (width 0.25) (layer "F.Cu") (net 35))
 (segment (start 135.825 87.685) (end 135.16 88.35) (width 0.25) (layer "F.Cu") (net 35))
 (segment (start 116.37137 89.84) (end 122.86 96.32863) (width 0.25) (layer "F.Cu") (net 34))
 (segment (start 122.86 96.32863) (end 122.86 97.46) (width 0.25) (layer "F.Cu") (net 34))
 (segment (start 115.24 89.84) (end 116.37137 89.84) (width 0.25) (layer "F.Cu") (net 34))
 (segment (start 123.9 97.46) (end 122.86 97.46) (width 0.25) (layer "B.Cu") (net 34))
 (segment (start 151.975 59.36) (end 149.53 59.36) (width 0.25) (layer "F.Cu") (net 30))
 (segment (start 149.53 59.36) (end 146.99 56.82) (width 0.25) (layer "F.Cu") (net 30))
 (segment (start 146.99 64.59) (end 151.825 64.59) (width 0.25) (layer "F.Cu") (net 31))
 (segment (start 151.825 64.59) (end 151.975 64.44) (width 0.25) (layer "F.Cu") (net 31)))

